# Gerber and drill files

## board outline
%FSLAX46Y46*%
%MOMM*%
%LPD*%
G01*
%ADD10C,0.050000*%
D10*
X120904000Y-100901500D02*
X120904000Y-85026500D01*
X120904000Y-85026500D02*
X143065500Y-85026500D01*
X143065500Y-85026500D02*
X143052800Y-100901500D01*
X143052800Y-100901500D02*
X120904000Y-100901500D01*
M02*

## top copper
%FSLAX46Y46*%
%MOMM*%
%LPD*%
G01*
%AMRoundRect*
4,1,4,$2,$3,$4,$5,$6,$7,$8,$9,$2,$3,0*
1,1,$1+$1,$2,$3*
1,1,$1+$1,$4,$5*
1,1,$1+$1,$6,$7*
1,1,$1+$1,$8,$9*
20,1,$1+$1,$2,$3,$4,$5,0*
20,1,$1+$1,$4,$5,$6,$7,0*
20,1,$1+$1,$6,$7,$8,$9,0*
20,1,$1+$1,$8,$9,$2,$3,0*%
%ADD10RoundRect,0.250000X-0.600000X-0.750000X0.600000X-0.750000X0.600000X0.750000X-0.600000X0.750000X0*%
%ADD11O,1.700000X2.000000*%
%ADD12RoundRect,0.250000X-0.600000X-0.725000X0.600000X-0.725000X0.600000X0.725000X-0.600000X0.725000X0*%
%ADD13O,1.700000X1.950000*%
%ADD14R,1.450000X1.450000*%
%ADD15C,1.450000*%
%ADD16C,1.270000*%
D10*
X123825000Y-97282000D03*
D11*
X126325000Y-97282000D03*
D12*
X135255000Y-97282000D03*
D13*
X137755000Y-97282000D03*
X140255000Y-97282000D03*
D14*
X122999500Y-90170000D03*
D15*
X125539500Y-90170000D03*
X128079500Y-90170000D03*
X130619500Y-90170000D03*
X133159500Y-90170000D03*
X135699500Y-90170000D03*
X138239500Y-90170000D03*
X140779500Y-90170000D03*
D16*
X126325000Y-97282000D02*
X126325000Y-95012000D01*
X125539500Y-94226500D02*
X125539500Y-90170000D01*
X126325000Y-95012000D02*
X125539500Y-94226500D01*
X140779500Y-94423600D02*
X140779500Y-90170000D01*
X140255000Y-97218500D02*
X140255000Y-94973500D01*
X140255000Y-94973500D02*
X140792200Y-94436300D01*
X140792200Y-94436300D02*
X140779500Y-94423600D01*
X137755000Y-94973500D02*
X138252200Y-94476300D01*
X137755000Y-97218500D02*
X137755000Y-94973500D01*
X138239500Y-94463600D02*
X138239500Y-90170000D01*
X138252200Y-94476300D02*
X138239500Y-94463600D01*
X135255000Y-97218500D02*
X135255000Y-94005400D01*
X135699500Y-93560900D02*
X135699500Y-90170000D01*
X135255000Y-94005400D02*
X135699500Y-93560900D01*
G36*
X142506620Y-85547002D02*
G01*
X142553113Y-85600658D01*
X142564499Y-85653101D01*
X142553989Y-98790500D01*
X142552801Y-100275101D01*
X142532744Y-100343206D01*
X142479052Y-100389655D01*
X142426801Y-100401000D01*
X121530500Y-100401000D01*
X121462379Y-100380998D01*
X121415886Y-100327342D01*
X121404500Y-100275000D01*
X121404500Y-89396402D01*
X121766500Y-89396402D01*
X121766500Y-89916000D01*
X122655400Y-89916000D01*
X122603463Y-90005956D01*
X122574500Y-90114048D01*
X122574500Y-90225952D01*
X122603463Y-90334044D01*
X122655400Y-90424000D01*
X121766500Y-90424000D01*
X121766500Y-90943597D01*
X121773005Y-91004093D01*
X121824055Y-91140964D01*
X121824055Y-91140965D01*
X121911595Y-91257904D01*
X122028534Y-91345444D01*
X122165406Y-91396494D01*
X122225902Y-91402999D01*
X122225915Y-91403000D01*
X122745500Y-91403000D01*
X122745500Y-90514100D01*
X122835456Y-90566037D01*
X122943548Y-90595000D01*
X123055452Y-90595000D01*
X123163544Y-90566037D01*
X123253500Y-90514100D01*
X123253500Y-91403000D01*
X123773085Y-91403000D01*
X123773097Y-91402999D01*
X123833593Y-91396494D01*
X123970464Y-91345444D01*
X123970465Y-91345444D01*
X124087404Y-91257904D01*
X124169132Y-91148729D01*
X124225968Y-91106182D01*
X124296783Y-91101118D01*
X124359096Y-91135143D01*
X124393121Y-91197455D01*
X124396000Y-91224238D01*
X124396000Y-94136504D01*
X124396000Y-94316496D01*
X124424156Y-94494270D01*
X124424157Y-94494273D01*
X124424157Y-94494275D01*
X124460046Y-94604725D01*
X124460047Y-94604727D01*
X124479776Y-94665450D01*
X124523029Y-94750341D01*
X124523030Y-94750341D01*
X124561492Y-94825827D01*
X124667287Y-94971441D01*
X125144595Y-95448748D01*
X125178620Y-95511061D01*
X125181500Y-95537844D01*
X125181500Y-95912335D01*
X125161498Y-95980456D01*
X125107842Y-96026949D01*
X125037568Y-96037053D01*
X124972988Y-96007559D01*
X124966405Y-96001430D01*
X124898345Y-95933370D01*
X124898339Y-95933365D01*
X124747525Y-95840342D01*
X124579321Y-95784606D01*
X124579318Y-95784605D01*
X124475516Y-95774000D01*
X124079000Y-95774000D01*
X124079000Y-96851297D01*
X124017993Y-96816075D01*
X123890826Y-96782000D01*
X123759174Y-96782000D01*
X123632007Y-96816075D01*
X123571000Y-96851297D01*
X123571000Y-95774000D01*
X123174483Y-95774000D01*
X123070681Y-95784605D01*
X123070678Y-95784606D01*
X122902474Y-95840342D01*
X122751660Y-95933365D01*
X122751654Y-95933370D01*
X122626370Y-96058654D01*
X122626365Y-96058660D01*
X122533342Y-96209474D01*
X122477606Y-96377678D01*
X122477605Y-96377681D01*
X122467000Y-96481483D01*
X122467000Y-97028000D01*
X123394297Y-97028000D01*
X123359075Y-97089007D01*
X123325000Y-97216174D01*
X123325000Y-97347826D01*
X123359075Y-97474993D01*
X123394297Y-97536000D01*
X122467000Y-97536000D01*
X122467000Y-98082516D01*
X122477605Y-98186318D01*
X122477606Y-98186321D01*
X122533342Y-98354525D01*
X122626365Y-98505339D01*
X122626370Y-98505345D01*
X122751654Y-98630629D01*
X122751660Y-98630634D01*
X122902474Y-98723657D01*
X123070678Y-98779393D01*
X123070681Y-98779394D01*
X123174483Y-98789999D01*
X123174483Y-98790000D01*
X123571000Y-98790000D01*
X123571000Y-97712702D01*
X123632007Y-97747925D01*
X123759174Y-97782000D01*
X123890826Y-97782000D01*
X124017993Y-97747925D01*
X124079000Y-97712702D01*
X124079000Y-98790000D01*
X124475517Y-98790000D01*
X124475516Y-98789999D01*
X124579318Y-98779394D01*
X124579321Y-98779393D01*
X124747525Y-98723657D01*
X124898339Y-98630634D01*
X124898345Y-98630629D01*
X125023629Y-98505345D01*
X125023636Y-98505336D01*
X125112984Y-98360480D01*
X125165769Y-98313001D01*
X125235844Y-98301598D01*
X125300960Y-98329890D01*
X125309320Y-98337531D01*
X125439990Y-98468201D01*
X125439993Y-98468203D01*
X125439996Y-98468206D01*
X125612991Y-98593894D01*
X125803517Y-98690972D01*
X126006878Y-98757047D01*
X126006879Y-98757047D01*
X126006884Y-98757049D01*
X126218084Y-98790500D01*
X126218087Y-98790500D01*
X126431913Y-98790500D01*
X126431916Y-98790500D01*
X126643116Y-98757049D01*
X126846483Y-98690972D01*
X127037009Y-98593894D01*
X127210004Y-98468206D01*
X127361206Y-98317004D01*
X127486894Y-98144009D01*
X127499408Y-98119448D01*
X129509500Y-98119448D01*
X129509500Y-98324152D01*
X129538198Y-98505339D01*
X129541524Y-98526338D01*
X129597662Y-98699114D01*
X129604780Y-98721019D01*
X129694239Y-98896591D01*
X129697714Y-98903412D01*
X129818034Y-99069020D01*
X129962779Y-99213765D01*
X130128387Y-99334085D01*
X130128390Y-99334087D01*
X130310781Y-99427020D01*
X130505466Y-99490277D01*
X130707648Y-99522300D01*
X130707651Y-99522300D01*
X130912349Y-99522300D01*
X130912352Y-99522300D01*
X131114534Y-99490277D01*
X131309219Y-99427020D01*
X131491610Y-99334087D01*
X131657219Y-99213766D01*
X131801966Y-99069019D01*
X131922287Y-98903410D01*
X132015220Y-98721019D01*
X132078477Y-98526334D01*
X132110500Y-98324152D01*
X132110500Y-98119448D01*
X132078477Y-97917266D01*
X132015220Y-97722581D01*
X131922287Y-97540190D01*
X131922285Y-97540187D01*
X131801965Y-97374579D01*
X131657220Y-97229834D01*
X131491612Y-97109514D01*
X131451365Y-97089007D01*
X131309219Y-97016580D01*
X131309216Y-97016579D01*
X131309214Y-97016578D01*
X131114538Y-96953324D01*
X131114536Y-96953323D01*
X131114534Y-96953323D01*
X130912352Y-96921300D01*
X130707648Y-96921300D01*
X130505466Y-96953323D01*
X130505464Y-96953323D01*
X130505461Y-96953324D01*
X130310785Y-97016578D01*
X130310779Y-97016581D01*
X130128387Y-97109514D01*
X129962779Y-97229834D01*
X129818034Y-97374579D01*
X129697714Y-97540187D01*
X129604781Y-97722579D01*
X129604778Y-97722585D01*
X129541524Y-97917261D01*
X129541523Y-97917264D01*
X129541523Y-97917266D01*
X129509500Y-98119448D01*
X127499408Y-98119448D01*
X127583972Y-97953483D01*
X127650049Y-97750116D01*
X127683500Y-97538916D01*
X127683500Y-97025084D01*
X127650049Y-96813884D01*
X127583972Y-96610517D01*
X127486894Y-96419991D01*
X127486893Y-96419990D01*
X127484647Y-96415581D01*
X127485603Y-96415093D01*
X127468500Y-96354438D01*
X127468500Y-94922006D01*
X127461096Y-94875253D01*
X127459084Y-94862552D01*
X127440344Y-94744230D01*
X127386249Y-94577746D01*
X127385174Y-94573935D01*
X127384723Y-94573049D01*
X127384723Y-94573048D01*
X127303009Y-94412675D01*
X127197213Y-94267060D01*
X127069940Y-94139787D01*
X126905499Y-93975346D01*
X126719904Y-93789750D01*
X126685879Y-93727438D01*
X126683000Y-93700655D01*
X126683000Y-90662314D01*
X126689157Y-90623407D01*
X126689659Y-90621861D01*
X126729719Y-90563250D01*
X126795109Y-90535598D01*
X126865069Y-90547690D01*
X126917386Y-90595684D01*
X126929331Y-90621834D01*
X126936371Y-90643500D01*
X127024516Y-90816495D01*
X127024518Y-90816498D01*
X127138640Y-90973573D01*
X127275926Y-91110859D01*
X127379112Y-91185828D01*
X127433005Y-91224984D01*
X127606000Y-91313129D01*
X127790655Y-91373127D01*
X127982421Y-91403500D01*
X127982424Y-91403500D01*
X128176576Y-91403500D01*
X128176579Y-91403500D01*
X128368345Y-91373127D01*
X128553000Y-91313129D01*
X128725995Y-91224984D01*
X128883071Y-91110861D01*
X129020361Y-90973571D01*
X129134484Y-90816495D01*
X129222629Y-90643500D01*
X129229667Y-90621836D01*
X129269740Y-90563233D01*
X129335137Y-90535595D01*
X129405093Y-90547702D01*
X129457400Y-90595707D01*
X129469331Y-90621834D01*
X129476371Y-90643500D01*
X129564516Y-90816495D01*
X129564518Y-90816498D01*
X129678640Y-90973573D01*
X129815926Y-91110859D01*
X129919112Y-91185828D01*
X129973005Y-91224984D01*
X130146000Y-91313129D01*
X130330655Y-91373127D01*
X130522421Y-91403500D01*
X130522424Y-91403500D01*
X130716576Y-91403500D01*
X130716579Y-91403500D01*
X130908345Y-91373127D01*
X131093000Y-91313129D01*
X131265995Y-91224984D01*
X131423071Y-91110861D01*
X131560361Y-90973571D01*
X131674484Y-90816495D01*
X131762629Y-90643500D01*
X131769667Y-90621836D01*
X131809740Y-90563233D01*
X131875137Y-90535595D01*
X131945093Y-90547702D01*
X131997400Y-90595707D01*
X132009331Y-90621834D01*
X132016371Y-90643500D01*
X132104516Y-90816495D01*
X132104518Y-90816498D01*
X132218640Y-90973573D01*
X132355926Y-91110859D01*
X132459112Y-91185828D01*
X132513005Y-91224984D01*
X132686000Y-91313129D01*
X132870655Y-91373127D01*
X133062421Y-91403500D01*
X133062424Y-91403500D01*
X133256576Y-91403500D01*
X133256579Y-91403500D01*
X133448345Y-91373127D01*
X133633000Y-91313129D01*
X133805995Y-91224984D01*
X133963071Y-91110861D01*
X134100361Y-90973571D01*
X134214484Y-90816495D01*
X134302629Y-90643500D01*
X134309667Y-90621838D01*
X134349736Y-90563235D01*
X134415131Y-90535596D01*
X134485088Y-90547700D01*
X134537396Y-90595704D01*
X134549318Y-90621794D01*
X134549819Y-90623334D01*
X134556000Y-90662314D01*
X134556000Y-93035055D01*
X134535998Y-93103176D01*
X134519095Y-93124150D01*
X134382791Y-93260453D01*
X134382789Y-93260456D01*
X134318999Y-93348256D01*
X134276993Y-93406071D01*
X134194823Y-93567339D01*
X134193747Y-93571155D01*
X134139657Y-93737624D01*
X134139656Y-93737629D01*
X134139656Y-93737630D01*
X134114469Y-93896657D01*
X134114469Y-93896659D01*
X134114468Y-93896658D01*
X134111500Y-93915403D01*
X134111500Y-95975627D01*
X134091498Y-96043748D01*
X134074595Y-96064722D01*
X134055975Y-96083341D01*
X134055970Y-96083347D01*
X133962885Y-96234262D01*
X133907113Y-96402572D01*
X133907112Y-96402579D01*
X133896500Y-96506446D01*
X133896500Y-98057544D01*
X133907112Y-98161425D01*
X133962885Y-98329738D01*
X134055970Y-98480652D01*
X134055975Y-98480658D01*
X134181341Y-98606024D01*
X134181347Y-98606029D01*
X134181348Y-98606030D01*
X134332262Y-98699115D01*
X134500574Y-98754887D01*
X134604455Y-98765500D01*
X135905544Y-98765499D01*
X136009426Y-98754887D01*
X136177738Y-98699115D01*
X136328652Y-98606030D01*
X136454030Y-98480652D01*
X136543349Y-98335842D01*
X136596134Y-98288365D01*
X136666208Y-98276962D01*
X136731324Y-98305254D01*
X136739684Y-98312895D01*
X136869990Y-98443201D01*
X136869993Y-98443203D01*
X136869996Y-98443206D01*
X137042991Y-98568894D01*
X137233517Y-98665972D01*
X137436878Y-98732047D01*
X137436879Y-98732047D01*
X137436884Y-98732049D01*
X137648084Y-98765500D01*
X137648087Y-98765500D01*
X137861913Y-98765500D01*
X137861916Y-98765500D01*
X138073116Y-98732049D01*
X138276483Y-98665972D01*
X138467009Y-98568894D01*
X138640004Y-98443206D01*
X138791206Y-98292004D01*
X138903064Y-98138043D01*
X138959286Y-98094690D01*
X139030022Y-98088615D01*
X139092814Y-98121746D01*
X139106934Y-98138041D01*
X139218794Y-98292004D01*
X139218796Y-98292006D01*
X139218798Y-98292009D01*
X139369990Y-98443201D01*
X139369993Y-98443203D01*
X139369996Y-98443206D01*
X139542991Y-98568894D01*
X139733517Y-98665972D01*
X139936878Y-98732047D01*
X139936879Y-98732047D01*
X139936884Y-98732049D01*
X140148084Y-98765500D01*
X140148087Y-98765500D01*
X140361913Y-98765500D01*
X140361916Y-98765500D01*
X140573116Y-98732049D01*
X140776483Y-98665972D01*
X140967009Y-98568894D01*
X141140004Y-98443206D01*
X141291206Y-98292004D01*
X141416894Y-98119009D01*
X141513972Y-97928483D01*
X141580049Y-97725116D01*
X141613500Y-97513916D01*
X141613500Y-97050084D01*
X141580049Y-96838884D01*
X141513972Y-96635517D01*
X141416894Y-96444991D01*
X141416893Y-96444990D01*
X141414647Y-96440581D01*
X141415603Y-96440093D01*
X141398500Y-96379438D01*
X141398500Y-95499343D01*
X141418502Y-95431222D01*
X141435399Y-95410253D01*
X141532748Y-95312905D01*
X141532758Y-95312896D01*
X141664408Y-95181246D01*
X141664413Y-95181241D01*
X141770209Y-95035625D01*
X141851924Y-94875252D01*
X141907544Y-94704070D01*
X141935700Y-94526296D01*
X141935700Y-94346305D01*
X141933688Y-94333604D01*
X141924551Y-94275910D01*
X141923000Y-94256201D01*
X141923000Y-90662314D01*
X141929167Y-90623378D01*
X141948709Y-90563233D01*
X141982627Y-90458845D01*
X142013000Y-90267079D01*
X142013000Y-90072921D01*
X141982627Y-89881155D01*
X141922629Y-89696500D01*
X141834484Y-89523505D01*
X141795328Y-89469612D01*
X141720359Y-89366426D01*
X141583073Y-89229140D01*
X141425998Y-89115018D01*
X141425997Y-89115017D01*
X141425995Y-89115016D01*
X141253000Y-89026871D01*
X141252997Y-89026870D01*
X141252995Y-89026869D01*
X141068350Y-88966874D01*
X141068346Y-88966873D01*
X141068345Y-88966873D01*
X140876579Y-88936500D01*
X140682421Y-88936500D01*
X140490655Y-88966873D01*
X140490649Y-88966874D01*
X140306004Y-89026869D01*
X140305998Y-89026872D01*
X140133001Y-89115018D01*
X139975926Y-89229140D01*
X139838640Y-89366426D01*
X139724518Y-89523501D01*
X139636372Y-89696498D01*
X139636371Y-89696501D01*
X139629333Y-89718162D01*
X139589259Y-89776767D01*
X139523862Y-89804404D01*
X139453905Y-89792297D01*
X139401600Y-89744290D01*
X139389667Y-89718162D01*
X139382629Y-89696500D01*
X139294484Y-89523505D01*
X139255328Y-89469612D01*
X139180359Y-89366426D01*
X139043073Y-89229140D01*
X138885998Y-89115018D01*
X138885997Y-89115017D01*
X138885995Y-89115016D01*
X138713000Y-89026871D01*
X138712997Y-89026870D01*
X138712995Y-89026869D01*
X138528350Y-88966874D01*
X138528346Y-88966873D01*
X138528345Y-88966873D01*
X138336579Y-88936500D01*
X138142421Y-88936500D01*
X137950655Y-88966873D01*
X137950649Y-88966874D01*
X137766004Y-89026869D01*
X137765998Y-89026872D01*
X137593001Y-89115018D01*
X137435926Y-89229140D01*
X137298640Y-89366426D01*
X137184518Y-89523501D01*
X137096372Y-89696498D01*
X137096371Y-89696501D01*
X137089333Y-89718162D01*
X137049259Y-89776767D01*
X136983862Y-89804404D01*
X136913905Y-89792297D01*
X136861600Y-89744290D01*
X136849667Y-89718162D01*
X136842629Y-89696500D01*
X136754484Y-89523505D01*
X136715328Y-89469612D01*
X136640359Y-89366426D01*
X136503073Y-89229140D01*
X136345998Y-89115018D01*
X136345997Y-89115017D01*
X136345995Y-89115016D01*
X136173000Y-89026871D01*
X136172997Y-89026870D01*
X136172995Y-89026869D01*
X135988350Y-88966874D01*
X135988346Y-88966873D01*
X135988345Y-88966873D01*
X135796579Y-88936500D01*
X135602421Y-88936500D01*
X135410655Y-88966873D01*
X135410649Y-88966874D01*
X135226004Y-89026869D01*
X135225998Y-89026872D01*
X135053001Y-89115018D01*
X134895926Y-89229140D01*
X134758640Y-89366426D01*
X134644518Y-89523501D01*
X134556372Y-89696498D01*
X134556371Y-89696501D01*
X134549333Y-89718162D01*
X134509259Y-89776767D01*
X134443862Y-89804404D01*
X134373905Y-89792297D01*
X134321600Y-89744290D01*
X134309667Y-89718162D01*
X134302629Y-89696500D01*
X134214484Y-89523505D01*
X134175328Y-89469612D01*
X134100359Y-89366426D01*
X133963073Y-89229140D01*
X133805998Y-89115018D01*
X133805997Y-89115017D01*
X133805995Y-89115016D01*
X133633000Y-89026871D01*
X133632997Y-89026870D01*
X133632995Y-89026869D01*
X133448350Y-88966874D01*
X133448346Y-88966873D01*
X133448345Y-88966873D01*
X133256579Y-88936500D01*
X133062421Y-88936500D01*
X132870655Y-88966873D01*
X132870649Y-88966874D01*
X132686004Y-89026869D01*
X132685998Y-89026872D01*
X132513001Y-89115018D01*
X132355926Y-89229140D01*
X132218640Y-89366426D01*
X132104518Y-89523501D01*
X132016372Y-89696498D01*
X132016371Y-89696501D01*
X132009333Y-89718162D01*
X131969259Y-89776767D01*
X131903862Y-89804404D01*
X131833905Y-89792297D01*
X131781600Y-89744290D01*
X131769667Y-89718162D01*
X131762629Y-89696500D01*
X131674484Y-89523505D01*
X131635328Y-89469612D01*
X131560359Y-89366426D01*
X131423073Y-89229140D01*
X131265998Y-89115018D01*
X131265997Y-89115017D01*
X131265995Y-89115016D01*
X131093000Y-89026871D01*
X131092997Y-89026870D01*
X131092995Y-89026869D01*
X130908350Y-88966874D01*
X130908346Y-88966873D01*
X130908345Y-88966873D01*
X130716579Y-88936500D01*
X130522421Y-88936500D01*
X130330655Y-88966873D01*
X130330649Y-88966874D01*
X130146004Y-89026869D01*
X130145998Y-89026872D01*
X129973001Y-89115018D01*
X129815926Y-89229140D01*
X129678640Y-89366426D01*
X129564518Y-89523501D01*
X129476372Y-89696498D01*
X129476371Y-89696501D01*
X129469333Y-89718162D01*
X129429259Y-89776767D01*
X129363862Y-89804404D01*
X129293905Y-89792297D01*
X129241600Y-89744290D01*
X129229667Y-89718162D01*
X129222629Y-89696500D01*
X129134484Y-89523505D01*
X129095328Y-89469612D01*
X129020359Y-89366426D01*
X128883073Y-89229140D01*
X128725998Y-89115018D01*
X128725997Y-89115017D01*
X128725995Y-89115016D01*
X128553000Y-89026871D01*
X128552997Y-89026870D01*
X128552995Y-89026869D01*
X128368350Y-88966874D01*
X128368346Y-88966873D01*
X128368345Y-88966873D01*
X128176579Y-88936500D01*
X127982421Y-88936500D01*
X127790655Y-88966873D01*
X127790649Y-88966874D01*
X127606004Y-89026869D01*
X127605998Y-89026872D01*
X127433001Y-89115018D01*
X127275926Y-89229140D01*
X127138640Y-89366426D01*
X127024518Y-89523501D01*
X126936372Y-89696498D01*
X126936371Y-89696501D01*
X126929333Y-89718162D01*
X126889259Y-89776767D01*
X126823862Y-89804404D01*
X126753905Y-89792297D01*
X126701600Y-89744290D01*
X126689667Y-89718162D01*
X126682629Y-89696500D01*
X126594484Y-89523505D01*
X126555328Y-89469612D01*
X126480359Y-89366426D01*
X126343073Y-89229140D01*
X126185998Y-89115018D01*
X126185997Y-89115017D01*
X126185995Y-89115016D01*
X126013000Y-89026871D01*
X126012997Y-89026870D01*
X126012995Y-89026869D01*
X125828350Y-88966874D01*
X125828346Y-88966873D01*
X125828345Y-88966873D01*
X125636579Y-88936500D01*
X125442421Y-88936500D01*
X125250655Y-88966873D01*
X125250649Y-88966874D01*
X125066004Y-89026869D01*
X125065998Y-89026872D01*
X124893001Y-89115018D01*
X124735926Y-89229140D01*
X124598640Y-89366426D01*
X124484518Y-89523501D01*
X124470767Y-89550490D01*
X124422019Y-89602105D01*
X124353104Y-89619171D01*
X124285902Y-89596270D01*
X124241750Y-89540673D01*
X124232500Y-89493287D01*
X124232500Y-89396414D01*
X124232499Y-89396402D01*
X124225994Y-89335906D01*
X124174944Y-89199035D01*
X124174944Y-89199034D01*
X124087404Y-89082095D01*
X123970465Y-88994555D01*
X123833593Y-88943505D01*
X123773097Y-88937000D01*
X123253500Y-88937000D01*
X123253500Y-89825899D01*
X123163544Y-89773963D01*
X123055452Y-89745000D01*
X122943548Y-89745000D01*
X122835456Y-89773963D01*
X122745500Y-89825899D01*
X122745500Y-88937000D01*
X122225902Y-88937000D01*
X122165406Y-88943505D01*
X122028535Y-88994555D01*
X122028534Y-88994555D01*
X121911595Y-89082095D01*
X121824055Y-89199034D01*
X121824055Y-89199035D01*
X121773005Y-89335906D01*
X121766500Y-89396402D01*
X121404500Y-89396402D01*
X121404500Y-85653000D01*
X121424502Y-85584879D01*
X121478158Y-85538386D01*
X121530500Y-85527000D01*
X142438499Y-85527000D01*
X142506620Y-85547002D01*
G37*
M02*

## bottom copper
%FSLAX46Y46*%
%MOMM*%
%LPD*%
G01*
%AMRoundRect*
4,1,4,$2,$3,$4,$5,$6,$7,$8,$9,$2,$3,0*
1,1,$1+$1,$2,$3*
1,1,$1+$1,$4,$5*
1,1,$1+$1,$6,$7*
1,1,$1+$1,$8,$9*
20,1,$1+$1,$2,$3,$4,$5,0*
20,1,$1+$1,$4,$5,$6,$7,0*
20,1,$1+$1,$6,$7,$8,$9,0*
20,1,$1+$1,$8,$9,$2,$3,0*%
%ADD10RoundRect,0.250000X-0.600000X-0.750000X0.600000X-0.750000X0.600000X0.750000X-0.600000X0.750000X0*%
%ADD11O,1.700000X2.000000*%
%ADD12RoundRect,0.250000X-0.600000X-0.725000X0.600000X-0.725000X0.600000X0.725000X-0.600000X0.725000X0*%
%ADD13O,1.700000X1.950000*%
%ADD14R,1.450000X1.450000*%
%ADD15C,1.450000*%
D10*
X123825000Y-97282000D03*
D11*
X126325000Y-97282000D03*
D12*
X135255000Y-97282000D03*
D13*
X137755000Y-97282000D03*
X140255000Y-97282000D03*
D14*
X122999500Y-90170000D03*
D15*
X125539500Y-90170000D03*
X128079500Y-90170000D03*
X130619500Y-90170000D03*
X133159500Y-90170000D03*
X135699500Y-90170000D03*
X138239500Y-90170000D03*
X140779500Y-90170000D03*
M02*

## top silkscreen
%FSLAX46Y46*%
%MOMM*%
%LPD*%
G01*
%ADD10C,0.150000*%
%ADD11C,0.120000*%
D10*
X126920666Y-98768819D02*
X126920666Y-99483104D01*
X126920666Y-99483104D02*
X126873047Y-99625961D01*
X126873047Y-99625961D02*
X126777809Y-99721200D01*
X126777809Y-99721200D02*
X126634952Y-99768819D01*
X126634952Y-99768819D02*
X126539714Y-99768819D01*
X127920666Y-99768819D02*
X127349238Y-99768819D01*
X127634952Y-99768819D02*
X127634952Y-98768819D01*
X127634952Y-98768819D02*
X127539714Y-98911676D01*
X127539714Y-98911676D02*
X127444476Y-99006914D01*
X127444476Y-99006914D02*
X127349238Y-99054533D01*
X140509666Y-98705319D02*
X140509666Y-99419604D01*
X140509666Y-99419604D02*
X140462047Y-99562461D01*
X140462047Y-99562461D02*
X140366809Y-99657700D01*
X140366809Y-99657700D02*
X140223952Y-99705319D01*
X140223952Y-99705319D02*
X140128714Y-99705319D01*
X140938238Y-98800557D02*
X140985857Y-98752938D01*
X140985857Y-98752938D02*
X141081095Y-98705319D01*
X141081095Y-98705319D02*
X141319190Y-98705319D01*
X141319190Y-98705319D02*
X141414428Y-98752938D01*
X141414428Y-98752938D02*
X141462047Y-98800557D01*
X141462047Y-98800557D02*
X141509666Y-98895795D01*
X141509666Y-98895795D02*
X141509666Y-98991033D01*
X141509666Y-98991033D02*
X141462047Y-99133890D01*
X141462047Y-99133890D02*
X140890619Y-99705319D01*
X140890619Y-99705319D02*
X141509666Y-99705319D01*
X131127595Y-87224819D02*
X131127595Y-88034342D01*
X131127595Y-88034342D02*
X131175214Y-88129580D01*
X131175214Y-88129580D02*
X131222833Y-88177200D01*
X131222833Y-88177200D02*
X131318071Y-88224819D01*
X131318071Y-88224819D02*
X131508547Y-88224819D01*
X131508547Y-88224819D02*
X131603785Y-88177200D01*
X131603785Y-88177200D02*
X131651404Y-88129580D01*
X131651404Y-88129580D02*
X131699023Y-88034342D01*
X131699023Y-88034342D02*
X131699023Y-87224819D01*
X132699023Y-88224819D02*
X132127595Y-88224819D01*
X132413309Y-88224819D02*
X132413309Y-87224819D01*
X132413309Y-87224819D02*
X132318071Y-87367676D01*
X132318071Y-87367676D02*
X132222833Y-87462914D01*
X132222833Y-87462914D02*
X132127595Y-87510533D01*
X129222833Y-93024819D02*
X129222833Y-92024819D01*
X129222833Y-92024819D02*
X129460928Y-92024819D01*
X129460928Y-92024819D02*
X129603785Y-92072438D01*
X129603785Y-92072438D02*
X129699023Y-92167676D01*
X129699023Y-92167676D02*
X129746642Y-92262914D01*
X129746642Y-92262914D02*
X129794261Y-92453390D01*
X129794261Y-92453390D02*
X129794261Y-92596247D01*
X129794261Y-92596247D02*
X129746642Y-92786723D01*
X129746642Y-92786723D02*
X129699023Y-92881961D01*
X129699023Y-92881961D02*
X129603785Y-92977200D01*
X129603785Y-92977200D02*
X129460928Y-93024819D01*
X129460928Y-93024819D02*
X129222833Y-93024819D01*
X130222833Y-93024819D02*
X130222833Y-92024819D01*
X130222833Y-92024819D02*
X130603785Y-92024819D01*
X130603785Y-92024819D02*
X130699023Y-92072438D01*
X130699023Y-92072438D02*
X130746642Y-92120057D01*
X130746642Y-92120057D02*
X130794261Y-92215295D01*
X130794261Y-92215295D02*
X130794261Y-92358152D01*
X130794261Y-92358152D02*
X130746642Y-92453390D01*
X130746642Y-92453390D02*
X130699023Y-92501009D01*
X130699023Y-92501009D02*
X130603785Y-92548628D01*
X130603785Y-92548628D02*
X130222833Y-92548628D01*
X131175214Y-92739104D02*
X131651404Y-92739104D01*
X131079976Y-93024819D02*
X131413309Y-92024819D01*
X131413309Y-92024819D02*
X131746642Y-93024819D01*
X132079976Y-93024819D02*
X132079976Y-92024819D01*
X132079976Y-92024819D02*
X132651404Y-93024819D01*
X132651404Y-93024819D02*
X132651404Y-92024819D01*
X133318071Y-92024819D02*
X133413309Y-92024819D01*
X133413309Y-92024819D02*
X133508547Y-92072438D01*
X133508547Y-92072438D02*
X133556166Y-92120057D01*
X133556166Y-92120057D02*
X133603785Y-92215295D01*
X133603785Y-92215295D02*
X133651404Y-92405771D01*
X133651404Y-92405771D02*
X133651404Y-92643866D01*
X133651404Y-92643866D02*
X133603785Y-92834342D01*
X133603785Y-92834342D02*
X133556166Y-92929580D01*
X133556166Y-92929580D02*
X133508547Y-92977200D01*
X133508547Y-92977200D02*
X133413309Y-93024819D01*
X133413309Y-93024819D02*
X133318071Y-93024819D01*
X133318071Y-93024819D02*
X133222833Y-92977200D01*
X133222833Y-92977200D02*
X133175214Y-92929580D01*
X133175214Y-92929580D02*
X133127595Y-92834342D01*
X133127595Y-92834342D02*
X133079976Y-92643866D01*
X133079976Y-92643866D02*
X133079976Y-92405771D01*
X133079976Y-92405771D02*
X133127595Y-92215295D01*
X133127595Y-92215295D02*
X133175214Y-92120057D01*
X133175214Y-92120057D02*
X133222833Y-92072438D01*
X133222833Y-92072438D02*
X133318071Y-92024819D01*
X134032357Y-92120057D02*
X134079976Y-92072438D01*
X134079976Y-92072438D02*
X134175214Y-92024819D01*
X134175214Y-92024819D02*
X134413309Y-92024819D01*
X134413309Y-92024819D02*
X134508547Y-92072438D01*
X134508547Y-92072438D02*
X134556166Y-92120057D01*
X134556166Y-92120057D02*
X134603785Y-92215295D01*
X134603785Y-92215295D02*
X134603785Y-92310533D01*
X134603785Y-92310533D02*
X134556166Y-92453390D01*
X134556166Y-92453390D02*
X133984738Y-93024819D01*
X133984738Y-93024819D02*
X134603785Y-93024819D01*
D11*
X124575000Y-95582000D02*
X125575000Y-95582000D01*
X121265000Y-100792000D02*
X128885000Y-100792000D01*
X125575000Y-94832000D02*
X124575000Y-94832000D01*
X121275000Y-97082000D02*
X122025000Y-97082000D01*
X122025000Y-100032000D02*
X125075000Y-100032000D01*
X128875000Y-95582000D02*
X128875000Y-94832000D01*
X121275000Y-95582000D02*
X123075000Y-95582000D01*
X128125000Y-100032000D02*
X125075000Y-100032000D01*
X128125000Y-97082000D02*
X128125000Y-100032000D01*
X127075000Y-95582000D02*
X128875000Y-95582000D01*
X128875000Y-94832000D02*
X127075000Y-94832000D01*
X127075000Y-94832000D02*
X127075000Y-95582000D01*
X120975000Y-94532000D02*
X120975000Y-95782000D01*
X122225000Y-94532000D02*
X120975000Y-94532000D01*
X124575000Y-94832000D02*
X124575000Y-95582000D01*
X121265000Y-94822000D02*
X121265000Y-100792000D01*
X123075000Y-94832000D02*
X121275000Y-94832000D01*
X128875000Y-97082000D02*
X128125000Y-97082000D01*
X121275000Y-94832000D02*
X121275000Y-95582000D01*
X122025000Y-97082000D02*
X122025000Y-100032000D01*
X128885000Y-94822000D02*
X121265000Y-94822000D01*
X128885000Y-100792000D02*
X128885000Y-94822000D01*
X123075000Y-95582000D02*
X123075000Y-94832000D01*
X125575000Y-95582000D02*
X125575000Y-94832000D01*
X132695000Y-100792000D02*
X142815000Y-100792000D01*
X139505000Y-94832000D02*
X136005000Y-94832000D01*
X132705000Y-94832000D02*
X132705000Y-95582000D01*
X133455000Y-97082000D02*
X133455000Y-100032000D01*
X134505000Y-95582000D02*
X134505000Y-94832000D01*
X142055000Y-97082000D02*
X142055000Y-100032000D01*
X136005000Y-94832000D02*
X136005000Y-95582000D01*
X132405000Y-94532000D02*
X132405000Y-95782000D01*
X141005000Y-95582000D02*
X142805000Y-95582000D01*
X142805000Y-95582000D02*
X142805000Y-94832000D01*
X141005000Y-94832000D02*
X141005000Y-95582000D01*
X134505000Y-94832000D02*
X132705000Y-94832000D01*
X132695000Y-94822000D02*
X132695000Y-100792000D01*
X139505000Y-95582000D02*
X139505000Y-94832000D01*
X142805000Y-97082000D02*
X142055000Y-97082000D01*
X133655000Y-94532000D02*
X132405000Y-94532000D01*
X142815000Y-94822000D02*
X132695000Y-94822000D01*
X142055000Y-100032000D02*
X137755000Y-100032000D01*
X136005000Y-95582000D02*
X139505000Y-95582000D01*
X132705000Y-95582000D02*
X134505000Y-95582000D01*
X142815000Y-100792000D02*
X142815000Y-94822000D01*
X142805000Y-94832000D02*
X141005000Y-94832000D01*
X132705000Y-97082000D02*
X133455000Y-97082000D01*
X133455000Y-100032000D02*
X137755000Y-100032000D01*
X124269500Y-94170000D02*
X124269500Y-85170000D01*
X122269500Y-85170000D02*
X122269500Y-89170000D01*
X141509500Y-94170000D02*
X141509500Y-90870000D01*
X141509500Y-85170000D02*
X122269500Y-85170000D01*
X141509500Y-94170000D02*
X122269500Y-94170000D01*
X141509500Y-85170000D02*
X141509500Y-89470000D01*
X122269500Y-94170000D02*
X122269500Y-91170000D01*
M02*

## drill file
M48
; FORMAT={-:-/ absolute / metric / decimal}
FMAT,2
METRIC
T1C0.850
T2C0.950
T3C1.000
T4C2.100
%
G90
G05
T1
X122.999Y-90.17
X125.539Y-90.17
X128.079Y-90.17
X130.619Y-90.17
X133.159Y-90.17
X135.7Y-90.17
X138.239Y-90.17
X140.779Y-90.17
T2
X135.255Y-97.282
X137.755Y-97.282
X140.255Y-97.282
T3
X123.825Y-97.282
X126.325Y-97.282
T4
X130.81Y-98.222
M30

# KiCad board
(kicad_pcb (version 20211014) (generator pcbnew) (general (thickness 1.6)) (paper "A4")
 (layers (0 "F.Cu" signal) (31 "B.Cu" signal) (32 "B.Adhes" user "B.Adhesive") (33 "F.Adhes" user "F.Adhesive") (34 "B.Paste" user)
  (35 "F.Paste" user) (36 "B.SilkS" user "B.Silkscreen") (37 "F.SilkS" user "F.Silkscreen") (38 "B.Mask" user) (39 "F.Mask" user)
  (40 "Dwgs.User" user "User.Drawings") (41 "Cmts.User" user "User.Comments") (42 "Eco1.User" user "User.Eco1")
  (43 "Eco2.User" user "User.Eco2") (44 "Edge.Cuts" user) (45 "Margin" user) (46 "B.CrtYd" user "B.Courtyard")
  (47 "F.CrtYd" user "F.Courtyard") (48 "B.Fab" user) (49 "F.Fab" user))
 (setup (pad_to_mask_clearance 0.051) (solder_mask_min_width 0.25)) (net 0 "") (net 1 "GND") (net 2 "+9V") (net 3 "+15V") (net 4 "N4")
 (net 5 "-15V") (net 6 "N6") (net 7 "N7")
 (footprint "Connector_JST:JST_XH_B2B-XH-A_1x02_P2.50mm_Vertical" (layer "F.Cu") (at 123.825 97.282)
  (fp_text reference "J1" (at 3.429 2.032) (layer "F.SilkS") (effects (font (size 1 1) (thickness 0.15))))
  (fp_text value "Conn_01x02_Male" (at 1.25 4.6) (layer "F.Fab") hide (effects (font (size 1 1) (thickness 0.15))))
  (fp_line (start 0.75 -1.7) (end 1.75 -1.7) (layer "F.SilkS") (width 0.12))
  (fp_line (start -2.56 3.51) (end 5.06 3.51) (layer "F.SilkS") (width 0.12))
  (fp_line (start 1.75 -2.45) (end 0.75 -2.45) (layer "F.SilkS") (width 0.12))
  (fp_line (start -2.55 -0.2) (end -1.8 -0.2) (layer "F.SilkS") (width 0.12))
  (fp_line (start -1.8 2.75) (end 1.25 2.75) (layer "F.SilkS") (width 0.12))
  (fp_line (start 5.05 -1.7) (end 5.05 -2.45) (layer "F.SilkS") (width 0.12))
  (fp_line (start -2.55 -1.7) (end -0.75 -1.7) (layer "F.SilkS") (width 0.12))
  (fp_line (start 4.3 2.75) (end 1.25 2.75) (layer "F.SilkS") (width 0.12))
  (fp_line (start 4.3 -0.2) (end 4.3 2.75) (layer "F.SilkS") (width 0.12))
  (fp_line (start 3.25 -1.7) (end 5.05 -1.7) (layer "F.SilkS") (width 0.12))
  (fp_line (start 5.05 -2.45) (end 3.25 -2.45) (layer "F.SilkS") (width 0.12))
  (fp_line (start 3.25 -2.45) (end 3.25 -1.7) (layer "F.SilkS") (width 0.12))
  (fp_line (start -2.85 -2.75) (end -2.85 -1.5) (layer "F.SilkS") (width 0.12))
  (fp_line (start -1.6 -2.75) (end -2.85 -2.75) (layer "F.SilkS") (width 0.12))
  (fp_line (start 0.75 -2.45) (end 0.75 -1.7) (layer "F.SilkS") (width 0.12))
  (fp_line (start -2.56 -2.46) (end -2.56 3.51) (layer "F.SilkS") (width 0.12))
  (fp_line (start -0.75 -2.45) (end -2.55 -2.45) (layer "F.SilkS") (width 0.12))
  (fp_line (start 5.05 -0.2) (end 4.3 -0.2) (layer "F.SilkS") (width 0.12))
  (fp_line (start -2.55 -2.45) (end -2.55 -1.7) (layer "F.SilkS") (width 0.12))
  (fp_line (start -1.8 -0.2) (end -1.8 2.75) (layer "F.SilkS") (width 0.12))
  (fp_line (start 5.06 -2.46) (end -2.56 -2.46) (layer "F.SilkS") (width 0.12))
  (fp_line (start 5.06 3.51) (end 5.06 -2.46) (layer "F.SilkS") (width 0.12))
  (fp_line (start -0.75 -1.7) (end -0.75 -2.45) (layer "F.SilkS") (width 0.12))
  (fp_line (start 1.75 -1.7) (end 1.75 -2.45) (layer "F.SilkS") (width 0.12))
  (pad "1" thru_hole roundrect locked (at 0 0) (size 1.7 2) (drill 1) (layers *.Cu *.Mask) (roundrect_rratio 0.147059) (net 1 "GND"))
  (pad "2" thru_hole oval locked (at 2.5 0) (size 1.7 2) (drill 1) (layers *.Cu *.Mask) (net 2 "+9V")))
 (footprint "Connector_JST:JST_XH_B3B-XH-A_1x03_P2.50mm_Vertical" (layer "F.Cu") (at 135.255 97.282)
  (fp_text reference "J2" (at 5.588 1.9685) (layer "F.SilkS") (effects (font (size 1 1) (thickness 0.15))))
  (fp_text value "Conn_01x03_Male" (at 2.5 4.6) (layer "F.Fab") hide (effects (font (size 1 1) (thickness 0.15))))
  (fp_line (start -2.56 3.51) (end 7.56 3.51) (layer "F.SilkS") (width 0.12))
  (fp_line (start 4.25 -2.45) (end 0.75 -2.45) (layer "F.SilkS") (width 0.12))
  (fp_line (start -2.55 -2.45) (end -2.55 -1.7) (layer "F.SilkS") (width 0.12))
  (fp_line (start -1.8 -0.2) (end -1.8 2.75) (layer "F.SilkS") (width 0.12))
  (fp_line (start -0.75 -1.7) (end -0.75 -2.45) (layer "F.SilkS") (width 0.12))
  (fp_line (start 6.8 -0.2) (end 6.8 2.75) (layer "F.SilkS") (width 0.12))
  (fp_line (start 0.75 -2.45) (end 0.75 -1.7) (layer "F.SilkS") (width 0.12))
  (fp_line (start -2.85 -2.75) (end -2.85 -1.5) (layer "F.SilkS") (width 0.12))
  (fp_line (start 5.75 -1.7) (end 7.55 -1.7) (layer "F.SilkS") (width 0.12))
  (fp_line (start 7.55 -1.7) (end 7.55 -2.45) (layer "F.SilkS") (width 0.12))
  (fp_line (start 5.75 -2.45) (end 5.75 -1.7) (layer "F.SilkS") (width 0.12))
  (fp_line (start -0.75 -2.45) (end -2.55 -2.45) (layer "F.SilkS") (width 0.12))
  (fp_line (start -2.56 -2.46) (end -2.56 3.51) (layer "F.SilkS") (width 0.12))
  (fp_line (start 4.25 -1.7) (end 4.25 -2.45) (layer "F.SilkS") (width 0.12))
  (fp_line (start 7.55 -0.2) (end 6.8 -0.2) (layer "F.SilkS") (width 0.12))
  (fp_line (start -1.6 -2.75) (end -2.85 -2.75) (layer "F.SilkS") (width 0.12))
  (fp_line (start 7.56 -2.46) (end -2.56 -2.46) (layer "F.SilkS") (width 0.12))
  (fp_line (start 6.8 2.75) (end 2.5 2.75) (layer "F.SilkS") (width 0.12))
  (fp_line (start 0.75 -1.7) (end 4.25 -1.7) (layer "F.SilkS") (width 0.12))
  (fp_line (start -2.55 -1.7) (end -0.75 -1.7) (layer "F.SilkS") (width 0.12))
  (fp_line (start 7.56 3.51) (end 7.56 -2.46) (layer "F.SilkS") (width 0.12))
  (fp_line (start 7.55 -2.45) (end 5.75 -2.45) (layer "F.SilkS") (width 0.12))
  (fp_line (start -2.55 -0.2) (end -1.8 -0.2) (layer "F.SilkS") (width 0.12))
  (fp_line (start -1.8 2.75) (end 2.5 2.75) (layer "F.SilkS") (width 0.12))
  (pad "1" thru_hole roundrect locked (at 0 0) (size 1.7 1.95) (drill 0.95) (layers *.Cu *.Mask) (roundrect_rratio 0.147059) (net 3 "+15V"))
  (pad "2" thru_hole oval locked (at 2.5 0) (size 1.7 1.95) (drill 0.95) (layers *.Cu *.Mask) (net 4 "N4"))
  (pad "3" thru_hole oval locked (at 5 0) (size 1.7 1.95) (drill 0.95) (layers *.Cu *.Mask) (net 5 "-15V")))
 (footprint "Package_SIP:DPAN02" (layer "F.Cu") (at 122.9995 90.17)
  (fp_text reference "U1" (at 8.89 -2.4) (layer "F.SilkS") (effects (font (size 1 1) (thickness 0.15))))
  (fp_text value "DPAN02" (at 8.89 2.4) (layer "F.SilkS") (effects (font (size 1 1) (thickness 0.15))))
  (fp_line (start 1.27 4) (end 1.27 -5) (layer "F.SilkS") (width 0.12))
  (fp_line (start -0.73 -5) (end -0.73 -1) (layer "F.SilkS") (width 0.12))
  (fp_line (start 18.51 4) (end 18.51 0.7) (layer "F.SilkS") (width 0.12))
  (fp_line (start 18.51 -5) (end -0.73 -5) (layer "F.SilkS") (width 0.12))
  (fp_line (start 18.51 4) (end -0.73 4) (layer "F.SilkS") (width 0.12))
  (fp_line (start 18.51 -5) (end 18.51 -0.7) (layer "F.SilkS") (width 0.12))
  (fp_line (start -0.73 4) (end -0.73 1) (layer "F.SilkS") (width 0.12))
  (pad "1" thru_hole rect locked (at 0 0 90) (size 1.45 1.45) (drill 0.85) (layers *.Cu *.Mask) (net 1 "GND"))
  (pad "2" thru_hole circle locked (at 2.54 0 90) (size 1.45 1.45) (drill 0.85) (layers *.Cu *.Mask) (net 2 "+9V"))
  (pad "3" thru_hole circle locked (at 5.08 0 90) (size 1.45 1.45) (drill 0.85) (layers *.Cu *.Mask) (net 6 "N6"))
  (pad "4" thru_hole circle locked (at 7.62 0 90) (size 1.45 1.45) (drill 0.85) (layers *.Cu *.Mask))
  (pad "5" thru_hole circle locked (at 10.16 0 90) (size 1.45 1.45) (drill 0.85) (layers *.Cu *.Mask) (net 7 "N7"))
  (pad "6" thru_hole circle locked (at 12.7 0 90) (size 1.45 1.45) (drill 0.85) (layers *.Cu *.Mask) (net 3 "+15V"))
  (pad "7" thru_hole circle locked (at 15.24 0 90) (size 1.45 1.45) (drill 0.85) (layers *.Cu *.Mask) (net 4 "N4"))
  (pad "8" thru_hole circle locked (at 17.78 0 90) (size 1.45 1.45) (drill 0.85) (layers *.Cu *.Mask) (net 5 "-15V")))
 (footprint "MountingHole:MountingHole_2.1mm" (layer "F.Cu") (at 130.81 98.2218)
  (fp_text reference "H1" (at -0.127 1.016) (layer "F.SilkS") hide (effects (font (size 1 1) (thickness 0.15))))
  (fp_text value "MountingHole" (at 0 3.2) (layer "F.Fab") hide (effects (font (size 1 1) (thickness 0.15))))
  (pad "" np_thru_hole circle locked (at 0 0) (size 2.1 2.1) (drill 2.1) (layers *.Cu *.Mask)))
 (gr_line (start 120.904 100.9015) (end 120.904 85.0265) (layer "Edge.Cuts") (width 0.05))
 (gr_line (start 120.904 85.0265) (end 143.0655 85.0265) (layer "Edge.Cuts") (width 0.05))
 (gr_line (start 143.0655 85.0265) (end 143.0528 100.9015) (layer "Edge.Cuts") (width 0.05))
 (gr_line (start 143.0528 100.9015) (end 120.904 100.9015) (layer "Edge.Cuts") (width 0.05))
 (segment (start 126.325 97.282) (end 126.325 95.012) (width 1.27) (layer "F.Cu") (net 2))
 (segment (start 125.5395 94.2265) (end 125.5395 90.17) (width 1.27) (layer "F.Cu") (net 2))
 (segment (start 126.325 95.012) (end 125.5395 94.2265) (width 1.27) (layer "F.Cu") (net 2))
 (segment (start 140.7795 94.4236) (end 140.7795 90.17) (width 1.27) (layer "F.Cu") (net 5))
 (segment (start 140.255 97.2185) (end 140.255 94.9735) (width 1.27) (layer "F.Cu") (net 5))
 (segment (start 140.255 94.9735) (end 140.7922 94.4363) (width 1.27) (layer "F.Cu") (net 5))
 (segment (start 140.7922 94.4363) (end 140.7795 94.4236) (width 1.27) (layer "F.Cu") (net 5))
 (segment (start 137.755 94.9735) (end 138.2522 94.4763) (width 1.27) (layer "F.Cu") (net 4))
 (segment (start 137.755 97.2185) (end 137.755 94.9735) (width 1.27) (layer "F.Cu") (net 4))
 (segment (start 138.2395 94.4636) (end 138.2395 90.17) (width 1.27) (layer "F.Cu") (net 4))
 (segment (start 138.2522 94.4763) (end 138.2395 94.4636) (width 1.27) (layer "F.Cu") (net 4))
 (segment (start 135.255 97.2185) (end 135.255 94.0054) (width 1.27) (layer "F.Cu") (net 3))
 (segment (start 135.6995 93.5609) (end 135.6995 90.17) (width 1.27) (layer "F.Cu") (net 3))
 (segment (start 135.255 94.0054) (end 135.6995 93.5609) (width 1.27) (layer "F.Cu") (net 3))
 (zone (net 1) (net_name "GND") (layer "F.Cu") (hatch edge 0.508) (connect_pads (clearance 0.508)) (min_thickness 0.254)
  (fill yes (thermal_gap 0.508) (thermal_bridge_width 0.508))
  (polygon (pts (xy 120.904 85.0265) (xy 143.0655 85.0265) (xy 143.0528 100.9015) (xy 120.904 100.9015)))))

